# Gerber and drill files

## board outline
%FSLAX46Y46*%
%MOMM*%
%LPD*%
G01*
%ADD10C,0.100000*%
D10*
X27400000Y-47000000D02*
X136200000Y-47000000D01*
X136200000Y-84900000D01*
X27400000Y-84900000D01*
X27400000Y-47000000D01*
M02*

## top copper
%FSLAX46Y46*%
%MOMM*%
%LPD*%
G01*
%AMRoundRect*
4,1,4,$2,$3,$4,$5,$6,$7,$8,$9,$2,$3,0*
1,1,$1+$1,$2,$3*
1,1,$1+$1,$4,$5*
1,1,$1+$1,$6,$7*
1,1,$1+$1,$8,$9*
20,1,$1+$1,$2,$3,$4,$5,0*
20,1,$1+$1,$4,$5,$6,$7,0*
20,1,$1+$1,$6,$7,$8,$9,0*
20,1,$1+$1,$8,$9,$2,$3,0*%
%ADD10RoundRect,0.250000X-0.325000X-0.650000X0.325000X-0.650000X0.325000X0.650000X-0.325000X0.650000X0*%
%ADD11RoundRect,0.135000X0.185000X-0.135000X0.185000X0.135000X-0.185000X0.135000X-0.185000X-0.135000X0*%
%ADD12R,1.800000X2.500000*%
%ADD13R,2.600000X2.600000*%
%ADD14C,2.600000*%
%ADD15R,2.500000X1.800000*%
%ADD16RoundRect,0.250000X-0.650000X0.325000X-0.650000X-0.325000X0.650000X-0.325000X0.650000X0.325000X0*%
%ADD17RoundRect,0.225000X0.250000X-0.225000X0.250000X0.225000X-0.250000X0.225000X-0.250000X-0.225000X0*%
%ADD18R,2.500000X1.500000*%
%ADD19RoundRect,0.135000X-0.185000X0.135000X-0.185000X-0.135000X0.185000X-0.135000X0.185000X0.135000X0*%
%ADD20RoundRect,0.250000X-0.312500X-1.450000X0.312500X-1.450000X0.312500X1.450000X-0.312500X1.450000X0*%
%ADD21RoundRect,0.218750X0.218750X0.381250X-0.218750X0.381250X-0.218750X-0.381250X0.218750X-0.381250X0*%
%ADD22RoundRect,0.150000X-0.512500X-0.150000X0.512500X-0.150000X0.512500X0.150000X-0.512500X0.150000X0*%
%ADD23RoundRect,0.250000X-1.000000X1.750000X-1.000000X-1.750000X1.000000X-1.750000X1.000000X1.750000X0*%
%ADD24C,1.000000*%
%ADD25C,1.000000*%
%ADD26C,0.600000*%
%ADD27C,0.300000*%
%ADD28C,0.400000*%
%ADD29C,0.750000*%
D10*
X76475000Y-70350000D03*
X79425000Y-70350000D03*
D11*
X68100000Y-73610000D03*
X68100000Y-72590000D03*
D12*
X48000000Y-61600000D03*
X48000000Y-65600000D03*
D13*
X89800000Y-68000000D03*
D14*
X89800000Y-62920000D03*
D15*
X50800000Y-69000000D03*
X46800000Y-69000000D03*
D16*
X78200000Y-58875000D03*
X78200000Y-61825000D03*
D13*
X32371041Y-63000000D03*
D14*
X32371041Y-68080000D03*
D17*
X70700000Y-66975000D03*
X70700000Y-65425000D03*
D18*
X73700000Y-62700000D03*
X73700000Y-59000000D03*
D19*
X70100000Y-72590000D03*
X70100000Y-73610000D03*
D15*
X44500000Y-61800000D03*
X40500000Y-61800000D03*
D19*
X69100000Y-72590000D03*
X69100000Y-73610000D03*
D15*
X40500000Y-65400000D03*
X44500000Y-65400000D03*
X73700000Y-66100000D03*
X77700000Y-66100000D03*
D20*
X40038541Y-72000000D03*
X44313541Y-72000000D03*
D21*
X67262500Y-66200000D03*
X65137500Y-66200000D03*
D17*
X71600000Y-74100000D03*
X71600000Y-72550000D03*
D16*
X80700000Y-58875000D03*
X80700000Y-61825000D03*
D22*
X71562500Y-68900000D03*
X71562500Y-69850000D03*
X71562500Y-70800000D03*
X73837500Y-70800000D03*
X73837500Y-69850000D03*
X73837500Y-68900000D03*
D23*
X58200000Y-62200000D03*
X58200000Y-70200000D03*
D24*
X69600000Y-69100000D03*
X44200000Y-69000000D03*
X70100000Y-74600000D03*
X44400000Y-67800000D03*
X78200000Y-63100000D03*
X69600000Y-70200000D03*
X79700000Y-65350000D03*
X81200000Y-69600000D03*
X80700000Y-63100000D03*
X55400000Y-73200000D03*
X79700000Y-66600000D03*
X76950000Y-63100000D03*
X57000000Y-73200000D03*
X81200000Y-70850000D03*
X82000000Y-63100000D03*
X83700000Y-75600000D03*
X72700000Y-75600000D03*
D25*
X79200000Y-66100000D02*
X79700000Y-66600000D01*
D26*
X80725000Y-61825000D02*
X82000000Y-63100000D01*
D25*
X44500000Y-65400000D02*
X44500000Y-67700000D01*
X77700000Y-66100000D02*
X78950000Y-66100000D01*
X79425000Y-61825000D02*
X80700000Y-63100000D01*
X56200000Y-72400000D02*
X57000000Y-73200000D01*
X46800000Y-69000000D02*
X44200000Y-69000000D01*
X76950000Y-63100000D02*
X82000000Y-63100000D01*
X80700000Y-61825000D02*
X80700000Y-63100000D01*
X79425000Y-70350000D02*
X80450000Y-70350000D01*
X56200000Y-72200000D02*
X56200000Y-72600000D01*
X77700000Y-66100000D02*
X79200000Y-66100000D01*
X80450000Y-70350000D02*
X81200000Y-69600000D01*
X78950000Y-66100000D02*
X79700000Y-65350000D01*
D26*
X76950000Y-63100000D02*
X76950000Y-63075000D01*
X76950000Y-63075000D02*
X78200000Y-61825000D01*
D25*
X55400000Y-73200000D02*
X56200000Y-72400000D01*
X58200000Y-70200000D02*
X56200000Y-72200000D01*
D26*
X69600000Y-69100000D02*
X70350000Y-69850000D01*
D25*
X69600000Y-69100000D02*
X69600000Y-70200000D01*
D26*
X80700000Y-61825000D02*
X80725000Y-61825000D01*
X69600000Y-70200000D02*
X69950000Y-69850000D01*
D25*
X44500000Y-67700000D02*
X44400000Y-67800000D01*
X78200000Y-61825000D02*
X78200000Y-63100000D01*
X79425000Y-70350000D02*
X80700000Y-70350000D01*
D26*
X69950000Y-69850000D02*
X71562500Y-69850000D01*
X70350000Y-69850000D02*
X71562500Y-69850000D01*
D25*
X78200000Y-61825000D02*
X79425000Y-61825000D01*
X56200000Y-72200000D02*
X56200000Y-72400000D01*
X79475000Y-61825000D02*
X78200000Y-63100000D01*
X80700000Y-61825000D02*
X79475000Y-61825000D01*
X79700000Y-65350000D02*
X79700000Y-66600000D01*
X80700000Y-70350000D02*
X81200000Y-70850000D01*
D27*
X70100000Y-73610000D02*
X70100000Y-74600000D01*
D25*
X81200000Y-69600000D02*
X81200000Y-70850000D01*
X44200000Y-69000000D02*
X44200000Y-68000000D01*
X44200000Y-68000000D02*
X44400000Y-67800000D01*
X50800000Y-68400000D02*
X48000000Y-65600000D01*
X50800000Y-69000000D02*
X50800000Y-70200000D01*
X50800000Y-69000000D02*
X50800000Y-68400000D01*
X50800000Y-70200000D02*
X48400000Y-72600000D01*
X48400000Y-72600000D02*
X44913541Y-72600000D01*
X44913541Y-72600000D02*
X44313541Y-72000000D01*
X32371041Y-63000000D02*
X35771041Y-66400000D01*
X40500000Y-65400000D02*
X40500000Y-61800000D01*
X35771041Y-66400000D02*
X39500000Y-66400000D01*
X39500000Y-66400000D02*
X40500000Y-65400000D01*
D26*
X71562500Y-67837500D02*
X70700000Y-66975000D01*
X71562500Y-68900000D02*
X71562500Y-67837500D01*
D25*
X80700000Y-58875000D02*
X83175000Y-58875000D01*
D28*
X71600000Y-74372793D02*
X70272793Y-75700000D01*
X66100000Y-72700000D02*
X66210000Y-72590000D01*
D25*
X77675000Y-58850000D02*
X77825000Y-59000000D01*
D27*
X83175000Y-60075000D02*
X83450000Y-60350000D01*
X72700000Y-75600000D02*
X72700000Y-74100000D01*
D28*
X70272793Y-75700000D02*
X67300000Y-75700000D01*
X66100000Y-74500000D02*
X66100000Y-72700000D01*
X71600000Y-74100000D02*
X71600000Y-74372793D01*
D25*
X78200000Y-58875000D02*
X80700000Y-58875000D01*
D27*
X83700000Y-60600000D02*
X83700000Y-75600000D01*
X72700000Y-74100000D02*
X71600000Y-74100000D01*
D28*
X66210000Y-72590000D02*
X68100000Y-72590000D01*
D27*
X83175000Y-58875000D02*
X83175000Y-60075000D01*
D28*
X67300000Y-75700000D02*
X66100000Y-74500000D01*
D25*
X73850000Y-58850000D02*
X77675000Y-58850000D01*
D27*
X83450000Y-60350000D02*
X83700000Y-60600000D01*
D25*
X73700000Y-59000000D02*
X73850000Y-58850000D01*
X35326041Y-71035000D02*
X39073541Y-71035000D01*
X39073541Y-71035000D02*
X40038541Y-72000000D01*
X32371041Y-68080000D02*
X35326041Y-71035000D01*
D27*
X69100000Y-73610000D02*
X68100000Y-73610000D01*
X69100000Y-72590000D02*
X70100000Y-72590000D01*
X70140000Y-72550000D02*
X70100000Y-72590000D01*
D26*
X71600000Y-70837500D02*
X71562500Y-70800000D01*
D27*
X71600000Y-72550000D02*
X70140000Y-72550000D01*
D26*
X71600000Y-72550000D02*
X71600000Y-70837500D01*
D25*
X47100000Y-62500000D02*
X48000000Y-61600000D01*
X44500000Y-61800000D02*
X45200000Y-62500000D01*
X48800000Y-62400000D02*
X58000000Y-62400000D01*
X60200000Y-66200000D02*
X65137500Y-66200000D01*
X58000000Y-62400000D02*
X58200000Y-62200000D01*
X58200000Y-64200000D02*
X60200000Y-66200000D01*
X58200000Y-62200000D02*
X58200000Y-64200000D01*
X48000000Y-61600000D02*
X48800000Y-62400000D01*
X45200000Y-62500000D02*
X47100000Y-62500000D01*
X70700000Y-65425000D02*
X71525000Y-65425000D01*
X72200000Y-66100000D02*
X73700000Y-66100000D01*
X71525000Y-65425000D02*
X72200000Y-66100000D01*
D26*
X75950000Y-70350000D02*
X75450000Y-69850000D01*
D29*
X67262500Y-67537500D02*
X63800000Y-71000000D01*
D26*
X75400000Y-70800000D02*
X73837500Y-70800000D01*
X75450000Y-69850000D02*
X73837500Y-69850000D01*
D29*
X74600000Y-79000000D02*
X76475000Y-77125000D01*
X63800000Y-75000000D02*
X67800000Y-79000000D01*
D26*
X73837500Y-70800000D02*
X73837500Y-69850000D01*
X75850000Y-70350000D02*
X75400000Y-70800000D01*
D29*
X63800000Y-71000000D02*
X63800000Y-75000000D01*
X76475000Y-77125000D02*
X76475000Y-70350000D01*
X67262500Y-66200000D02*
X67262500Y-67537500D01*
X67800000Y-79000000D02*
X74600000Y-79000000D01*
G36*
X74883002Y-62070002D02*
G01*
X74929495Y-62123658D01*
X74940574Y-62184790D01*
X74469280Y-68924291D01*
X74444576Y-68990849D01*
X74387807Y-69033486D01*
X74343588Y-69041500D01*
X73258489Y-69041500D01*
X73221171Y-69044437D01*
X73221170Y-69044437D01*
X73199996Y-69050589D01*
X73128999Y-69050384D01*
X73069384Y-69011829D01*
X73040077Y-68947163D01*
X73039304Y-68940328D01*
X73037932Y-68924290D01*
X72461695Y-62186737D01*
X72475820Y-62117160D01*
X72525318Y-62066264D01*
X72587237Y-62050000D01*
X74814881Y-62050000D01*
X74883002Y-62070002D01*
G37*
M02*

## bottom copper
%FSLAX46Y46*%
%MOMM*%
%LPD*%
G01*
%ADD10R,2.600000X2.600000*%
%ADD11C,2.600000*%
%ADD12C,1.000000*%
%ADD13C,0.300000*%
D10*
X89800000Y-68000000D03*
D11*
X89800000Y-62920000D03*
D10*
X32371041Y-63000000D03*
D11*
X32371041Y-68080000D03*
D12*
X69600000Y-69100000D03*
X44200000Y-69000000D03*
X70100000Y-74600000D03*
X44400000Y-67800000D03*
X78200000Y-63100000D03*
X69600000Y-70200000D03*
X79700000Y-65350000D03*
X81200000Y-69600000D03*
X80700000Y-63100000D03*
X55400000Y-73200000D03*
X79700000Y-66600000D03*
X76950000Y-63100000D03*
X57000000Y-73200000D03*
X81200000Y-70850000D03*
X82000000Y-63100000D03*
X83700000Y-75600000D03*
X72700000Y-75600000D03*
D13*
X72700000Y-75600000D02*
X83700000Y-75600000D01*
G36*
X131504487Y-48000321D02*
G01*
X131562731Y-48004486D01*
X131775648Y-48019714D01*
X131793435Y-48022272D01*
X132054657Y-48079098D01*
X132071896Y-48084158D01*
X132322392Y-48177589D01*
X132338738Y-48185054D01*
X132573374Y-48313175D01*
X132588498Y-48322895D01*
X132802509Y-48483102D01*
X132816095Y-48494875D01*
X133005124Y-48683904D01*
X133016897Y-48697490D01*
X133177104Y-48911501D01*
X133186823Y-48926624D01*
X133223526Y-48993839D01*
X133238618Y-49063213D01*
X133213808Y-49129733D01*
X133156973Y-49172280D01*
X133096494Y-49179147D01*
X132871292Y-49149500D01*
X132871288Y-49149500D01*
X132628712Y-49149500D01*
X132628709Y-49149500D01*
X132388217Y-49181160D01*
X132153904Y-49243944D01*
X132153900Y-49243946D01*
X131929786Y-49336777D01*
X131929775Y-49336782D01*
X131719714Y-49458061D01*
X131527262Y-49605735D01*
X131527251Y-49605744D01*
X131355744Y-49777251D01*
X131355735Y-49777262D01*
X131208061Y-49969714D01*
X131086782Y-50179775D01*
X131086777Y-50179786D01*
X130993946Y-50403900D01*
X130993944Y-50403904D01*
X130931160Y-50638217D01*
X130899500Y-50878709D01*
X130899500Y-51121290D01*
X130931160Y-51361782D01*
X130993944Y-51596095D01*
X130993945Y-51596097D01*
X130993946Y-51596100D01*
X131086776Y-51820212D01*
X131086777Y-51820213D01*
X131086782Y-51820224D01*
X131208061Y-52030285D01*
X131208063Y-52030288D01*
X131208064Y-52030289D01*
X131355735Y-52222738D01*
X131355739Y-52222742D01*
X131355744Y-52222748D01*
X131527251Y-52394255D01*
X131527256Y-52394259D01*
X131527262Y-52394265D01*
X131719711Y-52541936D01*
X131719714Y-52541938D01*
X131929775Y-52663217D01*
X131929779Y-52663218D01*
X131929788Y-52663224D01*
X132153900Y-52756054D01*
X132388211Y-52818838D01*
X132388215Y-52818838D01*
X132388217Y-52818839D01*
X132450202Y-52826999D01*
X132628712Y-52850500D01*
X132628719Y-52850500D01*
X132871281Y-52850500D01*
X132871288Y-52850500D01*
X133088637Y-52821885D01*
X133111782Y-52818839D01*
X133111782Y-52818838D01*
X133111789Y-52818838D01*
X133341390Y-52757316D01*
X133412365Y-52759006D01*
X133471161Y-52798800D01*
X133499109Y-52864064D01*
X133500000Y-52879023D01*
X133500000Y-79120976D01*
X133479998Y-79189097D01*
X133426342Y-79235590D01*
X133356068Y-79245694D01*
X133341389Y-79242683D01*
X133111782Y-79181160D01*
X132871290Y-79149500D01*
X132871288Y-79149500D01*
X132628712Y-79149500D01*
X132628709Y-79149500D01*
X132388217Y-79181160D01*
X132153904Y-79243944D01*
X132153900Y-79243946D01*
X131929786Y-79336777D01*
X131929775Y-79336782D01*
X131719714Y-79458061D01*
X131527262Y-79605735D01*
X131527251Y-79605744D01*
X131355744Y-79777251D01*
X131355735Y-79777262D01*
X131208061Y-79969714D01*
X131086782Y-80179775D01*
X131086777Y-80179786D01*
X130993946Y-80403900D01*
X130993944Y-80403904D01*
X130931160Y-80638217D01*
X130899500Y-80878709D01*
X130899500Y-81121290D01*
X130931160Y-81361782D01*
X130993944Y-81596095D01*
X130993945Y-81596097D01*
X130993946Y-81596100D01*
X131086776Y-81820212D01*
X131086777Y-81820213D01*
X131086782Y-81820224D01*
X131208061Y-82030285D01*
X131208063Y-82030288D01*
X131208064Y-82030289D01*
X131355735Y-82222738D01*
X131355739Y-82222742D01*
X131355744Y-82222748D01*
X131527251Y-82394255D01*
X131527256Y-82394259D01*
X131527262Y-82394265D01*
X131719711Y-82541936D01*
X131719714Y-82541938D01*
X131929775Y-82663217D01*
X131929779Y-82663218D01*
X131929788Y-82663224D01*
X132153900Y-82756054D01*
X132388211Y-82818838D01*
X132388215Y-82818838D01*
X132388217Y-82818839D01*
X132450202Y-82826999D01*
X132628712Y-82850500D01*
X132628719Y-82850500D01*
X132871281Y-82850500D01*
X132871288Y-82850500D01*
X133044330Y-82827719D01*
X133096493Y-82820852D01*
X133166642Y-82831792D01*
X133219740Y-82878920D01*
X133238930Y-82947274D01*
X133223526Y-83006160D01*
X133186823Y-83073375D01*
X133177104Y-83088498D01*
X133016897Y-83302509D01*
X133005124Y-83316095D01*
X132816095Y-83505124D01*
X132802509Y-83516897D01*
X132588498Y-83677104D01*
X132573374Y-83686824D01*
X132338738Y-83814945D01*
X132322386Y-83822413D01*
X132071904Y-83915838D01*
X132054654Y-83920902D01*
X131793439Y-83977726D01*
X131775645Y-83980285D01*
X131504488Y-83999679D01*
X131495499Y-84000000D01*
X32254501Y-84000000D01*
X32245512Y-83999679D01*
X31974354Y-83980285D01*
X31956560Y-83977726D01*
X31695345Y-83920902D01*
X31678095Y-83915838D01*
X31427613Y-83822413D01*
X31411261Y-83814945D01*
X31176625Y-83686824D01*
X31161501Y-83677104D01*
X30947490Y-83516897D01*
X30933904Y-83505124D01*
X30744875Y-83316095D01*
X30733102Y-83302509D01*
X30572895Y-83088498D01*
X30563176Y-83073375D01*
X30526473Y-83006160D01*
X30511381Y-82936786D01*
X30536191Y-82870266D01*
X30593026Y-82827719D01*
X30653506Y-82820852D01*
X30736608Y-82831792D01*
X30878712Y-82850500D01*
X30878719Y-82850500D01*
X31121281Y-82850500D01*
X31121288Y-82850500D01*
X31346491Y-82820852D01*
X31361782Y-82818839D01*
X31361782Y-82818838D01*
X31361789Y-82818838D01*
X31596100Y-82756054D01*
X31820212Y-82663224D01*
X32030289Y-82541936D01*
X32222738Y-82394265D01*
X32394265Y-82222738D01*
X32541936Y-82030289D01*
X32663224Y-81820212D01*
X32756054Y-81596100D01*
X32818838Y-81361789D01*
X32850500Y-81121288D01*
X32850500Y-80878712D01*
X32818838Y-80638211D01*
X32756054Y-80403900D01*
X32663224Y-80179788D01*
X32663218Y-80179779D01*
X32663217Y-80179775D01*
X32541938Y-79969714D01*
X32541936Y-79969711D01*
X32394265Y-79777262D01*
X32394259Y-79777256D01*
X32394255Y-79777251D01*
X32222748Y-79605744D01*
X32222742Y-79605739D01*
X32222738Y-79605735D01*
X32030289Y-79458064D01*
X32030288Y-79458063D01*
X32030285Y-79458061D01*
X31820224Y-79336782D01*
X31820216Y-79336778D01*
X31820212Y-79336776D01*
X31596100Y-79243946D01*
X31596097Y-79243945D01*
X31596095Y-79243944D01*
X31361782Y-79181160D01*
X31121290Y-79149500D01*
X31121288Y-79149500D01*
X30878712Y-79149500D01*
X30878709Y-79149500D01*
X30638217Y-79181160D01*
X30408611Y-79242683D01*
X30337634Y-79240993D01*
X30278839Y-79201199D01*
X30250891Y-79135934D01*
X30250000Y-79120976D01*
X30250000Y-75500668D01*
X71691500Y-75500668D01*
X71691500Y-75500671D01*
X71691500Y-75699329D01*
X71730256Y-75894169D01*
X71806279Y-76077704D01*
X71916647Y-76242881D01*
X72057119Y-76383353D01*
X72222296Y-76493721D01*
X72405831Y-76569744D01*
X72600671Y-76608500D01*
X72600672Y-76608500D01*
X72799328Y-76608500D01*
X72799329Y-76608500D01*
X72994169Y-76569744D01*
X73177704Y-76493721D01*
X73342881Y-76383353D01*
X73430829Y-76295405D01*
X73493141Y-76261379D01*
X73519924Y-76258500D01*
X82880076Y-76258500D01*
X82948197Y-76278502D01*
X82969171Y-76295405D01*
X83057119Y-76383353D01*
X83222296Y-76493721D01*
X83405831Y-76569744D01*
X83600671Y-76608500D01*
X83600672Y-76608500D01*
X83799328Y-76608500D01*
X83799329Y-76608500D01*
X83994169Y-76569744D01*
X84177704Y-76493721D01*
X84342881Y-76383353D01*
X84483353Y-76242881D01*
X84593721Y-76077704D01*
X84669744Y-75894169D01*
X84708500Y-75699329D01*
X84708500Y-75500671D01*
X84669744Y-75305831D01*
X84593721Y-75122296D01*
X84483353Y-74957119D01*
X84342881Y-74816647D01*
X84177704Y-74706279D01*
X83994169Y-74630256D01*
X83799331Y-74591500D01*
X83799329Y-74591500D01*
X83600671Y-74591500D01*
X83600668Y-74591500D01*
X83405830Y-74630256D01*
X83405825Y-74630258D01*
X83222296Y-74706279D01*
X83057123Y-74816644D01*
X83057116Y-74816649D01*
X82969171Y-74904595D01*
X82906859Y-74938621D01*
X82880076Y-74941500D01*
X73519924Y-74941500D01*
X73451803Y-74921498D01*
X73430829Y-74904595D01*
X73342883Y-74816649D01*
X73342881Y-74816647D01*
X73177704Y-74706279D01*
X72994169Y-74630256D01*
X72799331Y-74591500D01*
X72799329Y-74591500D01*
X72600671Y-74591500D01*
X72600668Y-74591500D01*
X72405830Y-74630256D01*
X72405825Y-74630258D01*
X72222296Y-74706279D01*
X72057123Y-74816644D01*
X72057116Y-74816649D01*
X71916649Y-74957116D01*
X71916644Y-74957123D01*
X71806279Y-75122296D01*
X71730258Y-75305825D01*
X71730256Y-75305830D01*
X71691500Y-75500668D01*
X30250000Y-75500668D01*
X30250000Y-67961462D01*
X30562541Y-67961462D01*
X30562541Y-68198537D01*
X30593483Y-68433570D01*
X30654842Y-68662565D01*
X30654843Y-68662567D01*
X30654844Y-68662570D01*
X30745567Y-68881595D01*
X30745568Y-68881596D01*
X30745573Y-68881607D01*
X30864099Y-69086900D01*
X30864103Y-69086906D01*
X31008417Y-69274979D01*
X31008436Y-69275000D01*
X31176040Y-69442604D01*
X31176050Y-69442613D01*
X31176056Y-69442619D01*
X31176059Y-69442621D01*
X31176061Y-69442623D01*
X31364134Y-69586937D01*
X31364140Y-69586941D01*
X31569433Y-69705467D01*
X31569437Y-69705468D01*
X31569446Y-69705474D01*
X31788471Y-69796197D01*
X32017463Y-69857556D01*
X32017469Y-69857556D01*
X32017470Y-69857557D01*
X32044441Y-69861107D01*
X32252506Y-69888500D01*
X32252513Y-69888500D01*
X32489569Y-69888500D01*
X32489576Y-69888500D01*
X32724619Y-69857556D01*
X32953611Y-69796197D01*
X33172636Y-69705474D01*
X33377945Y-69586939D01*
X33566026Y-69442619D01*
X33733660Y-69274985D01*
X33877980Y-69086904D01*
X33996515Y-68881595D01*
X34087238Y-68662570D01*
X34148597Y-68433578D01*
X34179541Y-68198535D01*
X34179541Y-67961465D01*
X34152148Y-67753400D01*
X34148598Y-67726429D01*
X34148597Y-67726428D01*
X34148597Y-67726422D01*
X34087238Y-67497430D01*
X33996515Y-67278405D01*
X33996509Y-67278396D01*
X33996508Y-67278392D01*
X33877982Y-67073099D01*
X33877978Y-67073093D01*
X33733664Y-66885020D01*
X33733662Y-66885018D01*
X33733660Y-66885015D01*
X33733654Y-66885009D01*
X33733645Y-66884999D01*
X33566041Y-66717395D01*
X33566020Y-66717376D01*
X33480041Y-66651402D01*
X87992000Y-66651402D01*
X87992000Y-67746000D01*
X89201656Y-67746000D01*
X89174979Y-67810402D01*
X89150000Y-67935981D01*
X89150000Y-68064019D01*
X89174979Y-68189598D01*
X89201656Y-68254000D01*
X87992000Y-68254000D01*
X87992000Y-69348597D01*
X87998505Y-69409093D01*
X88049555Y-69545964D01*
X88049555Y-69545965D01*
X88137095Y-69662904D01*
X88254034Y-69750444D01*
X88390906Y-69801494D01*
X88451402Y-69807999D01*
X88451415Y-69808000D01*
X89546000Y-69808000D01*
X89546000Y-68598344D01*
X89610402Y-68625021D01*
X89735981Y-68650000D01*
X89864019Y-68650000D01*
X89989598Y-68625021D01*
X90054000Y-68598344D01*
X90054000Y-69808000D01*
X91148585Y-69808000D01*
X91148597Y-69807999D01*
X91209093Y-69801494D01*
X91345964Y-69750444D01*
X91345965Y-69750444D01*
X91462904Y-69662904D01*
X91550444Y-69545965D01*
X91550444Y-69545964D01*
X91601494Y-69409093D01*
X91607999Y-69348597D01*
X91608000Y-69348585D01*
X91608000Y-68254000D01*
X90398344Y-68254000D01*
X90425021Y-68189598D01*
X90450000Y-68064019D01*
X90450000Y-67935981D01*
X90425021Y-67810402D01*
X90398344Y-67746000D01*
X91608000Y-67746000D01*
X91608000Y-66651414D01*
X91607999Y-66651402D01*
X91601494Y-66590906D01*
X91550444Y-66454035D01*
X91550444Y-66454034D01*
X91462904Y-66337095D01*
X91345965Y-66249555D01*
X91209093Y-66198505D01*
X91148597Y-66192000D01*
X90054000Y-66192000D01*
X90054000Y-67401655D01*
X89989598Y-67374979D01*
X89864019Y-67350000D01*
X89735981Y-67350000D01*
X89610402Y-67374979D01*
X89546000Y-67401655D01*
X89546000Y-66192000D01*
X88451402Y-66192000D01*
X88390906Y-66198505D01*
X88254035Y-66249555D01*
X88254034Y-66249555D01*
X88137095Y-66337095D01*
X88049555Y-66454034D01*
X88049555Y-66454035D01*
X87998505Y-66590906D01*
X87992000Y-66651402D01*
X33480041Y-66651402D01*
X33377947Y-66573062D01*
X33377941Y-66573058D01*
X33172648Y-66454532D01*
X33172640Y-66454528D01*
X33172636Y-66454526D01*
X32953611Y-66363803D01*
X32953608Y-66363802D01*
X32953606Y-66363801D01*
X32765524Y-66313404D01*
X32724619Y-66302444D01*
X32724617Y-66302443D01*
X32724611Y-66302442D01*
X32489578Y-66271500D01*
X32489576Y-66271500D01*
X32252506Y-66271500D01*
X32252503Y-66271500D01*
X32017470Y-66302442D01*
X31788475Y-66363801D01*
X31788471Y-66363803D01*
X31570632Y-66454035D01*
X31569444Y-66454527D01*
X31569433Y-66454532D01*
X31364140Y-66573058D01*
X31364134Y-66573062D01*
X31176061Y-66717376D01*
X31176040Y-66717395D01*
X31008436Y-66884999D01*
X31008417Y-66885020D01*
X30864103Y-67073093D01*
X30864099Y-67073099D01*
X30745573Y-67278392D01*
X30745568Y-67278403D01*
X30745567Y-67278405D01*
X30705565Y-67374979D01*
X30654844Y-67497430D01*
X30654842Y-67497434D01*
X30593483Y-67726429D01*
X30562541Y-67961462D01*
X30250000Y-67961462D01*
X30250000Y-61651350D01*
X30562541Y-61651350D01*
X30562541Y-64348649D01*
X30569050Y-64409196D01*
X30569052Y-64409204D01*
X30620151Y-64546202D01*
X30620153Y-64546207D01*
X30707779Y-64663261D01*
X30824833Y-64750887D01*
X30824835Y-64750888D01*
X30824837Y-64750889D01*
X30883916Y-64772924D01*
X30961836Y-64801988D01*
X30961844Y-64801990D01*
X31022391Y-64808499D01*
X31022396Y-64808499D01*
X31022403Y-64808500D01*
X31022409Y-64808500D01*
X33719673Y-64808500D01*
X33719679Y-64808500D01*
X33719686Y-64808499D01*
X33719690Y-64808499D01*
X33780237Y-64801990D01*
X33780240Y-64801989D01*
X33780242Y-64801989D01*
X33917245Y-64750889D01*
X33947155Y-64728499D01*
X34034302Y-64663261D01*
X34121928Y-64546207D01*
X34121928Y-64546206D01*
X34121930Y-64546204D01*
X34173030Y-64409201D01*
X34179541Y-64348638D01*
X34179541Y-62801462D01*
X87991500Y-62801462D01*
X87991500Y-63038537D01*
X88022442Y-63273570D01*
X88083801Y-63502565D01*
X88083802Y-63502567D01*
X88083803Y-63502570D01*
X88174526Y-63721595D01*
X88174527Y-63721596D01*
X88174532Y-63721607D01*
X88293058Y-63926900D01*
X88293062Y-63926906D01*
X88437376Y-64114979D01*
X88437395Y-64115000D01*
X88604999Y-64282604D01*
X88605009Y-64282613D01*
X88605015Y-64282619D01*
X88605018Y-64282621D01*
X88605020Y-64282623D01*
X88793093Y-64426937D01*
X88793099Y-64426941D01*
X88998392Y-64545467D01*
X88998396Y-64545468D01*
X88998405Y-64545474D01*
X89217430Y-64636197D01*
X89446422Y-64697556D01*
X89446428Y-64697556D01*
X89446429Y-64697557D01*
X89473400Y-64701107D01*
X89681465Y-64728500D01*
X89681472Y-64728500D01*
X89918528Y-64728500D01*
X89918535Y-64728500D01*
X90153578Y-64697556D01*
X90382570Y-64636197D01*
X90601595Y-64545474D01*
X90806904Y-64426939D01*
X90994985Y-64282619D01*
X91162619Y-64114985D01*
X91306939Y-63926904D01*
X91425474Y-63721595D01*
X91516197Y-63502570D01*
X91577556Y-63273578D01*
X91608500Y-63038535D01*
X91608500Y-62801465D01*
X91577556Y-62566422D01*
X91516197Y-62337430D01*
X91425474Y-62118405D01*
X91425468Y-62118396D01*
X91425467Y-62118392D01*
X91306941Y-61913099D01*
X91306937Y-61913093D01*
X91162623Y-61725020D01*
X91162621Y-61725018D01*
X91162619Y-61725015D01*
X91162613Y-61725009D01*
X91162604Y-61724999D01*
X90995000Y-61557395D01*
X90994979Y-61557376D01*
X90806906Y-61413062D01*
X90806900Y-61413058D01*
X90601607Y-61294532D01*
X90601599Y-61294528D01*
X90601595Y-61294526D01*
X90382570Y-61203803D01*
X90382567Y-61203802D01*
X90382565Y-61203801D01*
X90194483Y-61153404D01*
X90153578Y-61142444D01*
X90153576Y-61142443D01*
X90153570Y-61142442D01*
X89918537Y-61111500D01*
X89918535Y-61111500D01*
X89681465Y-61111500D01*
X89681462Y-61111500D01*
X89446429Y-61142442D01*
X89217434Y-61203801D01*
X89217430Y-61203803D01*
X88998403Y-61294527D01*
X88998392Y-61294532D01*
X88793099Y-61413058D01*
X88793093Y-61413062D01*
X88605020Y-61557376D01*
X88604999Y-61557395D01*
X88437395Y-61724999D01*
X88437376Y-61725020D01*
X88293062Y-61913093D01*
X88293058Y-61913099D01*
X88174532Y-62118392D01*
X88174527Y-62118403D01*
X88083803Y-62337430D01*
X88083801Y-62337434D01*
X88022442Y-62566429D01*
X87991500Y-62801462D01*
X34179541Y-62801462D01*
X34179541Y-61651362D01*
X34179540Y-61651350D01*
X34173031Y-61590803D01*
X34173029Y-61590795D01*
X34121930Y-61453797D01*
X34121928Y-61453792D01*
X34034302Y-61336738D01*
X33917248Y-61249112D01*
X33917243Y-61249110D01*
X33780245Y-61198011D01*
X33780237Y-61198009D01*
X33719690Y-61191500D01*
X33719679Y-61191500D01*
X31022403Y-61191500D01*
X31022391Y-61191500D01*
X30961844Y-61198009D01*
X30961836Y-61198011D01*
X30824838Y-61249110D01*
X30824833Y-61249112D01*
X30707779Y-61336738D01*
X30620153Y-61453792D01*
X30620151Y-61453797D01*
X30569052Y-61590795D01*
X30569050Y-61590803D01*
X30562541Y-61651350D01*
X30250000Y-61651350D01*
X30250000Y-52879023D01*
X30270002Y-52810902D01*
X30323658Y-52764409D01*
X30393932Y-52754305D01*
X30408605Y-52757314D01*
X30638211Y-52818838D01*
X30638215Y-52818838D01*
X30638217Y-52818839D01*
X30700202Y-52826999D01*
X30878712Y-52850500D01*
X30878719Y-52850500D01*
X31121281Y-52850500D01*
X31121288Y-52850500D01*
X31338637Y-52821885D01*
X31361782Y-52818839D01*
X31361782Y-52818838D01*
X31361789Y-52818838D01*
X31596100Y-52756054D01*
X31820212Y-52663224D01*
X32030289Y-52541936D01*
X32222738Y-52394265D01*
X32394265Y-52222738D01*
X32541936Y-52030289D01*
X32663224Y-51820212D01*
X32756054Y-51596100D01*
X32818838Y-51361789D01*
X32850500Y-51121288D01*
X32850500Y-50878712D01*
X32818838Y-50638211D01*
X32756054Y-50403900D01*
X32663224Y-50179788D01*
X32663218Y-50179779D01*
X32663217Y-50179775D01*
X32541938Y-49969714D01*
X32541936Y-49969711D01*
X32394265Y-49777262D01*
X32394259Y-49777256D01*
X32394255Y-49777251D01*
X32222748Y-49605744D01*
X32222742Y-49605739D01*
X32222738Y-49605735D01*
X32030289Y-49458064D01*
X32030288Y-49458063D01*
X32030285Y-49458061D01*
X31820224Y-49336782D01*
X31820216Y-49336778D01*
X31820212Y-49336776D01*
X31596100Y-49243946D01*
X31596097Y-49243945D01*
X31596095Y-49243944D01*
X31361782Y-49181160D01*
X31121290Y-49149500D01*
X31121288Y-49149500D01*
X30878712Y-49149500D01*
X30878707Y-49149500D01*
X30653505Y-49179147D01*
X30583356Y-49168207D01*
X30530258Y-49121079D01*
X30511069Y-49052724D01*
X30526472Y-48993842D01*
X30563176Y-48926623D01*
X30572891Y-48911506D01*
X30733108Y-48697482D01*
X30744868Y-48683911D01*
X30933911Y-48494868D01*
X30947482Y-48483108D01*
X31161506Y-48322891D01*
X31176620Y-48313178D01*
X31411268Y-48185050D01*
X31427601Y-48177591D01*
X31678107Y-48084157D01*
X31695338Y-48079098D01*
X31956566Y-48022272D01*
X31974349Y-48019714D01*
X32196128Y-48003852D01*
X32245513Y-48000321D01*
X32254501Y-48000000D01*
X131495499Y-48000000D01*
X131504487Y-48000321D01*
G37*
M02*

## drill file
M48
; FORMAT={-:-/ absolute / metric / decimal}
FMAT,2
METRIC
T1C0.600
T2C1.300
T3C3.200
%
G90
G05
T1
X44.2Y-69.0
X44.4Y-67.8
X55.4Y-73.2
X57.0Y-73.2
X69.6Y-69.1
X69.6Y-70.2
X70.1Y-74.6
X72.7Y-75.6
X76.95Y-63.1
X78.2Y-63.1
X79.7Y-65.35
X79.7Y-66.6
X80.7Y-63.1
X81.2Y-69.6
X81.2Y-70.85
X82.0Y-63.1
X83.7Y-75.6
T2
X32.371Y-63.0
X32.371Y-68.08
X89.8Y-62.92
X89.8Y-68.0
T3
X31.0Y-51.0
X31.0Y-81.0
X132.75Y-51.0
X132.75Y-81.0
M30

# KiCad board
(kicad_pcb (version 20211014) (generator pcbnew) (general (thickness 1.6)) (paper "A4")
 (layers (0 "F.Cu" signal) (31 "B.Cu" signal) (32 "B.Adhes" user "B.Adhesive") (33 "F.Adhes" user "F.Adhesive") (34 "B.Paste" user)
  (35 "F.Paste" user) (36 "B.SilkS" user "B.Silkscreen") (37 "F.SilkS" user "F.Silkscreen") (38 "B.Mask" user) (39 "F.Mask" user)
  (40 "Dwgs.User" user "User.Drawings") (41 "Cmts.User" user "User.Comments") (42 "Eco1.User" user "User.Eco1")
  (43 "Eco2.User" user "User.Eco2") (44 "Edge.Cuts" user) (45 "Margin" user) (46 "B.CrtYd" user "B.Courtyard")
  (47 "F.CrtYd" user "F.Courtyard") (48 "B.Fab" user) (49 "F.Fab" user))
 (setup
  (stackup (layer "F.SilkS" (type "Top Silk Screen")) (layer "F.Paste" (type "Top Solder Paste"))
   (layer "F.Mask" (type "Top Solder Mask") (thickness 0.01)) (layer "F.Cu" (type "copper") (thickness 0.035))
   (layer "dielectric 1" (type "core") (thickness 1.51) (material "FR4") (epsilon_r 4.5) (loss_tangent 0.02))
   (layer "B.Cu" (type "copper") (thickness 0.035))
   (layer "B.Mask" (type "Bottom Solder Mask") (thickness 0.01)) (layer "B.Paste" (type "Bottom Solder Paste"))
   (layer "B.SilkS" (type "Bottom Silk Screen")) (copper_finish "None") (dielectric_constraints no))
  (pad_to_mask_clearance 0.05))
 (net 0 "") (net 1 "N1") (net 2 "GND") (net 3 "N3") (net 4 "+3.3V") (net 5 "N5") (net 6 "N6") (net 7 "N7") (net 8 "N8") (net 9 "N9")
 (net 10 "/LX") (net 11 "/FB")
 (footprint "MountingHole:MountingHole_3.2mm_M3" (layer "F.Cu") (at 132.75 51)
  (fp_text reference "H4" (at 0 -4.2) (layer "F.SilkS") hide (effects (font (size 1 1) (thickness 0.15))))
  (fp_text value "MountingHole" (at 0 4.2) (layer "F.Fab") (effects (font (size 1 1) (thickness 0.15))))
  (pad "" np_thru_hole circle (at 0 0) (size 3.2 3.2) (drill 3.2) (layers *.Cu *.Mask)))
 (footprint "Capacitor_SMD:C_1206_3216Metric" (layer "F.Cu") (at 77.95 70.35)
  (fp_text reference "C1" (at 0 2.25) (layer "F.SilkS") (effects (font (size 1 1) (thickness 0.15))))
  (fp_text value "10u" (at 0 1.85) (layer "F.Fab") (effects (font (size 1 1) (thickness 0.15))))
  (pad "1" smd roundrect (at -1.475 0) (size 1.15 1.8) (layers "F.Cu" "F.Paste" "F.Mask") (roundrect_rratio 0.217391) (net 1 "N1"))
  (pad "2" smd roundrect (at 1.475 0) (size 1.15 1.8) (layers "F.Cu" "F.Paste" "F.Mask") (roundrect_rratio 0.217391) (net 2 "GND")))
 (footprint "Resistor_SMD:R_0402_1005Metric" (layer "F.Cu") (at 68.1 73.1 90)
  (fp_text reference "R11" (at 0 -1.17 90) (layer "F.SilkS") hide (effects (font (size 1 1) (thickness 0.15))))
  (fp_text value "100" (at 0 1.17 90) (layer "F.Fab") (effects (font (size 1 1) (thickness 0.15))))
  (pad "1" smd roundrect (at -0.51 0 90) (size 0.54 0.64) (layers "F.Cu" "F.Paste" "F.Mask") (roundrect_rratio 0.25) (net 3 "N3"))
  (pad "2" smd roundrect (at 0.51 0 90) (size 0.54 0.64) (layers "F.Cu" "F.Paste" "F.Mask") (roundrect_rratio 0.25) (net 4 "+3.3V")))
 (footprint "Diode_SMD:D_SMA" (layer "F.Cu") (at 48 63.6 -90)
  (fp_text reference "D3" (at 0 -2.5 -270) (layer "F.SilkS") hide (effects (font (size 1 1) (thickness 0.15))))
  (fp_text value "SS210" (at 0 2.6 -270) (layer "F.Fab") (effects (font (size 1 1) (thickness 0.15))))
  (pad "1" smd rect (at -2 0 270) (size 2.5 1.8) (layers "F.Cu" "F.Paste" "F.Mask") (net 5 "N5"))
  (pad "2" smd rect (at 2 0 270) (size 2.5 1.8) (layers "F.Cu" "F.Paste" "F.Mask") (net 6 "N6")))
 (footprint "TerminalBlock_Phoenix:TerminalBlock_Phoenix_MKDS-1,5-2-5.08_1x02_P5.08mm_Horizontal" (layer "F.Cu") (at 89.8 68 90)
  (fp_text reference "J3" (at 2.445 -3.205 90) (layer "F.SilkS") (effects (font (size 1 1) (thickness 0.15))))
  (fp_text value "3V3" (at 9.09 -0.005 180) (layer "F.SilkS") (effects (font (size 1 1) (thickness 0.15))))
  (pad "1" thru_hole rect (at 0 0 90) (size 2.6 2.6) (drill 1.3) (layers *.Cu *.Mask) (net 2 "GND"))
  (pad "2" thru_hole circle (at 5.08 0 90) (size 2.6 2.6) (drill 1.3) (layers *.Cu *.Mask) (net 4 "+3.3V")))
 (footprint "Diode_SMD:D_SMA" (layer "F.Cu") (at 48.8 69 180)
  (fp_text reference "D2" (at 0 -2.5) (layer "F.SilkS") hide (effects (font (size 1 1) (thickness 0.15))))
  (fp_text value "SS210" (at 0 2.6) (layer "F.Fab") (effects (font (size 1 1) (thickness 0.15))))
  (pad "1" smd rect (at -2 0 180) (size 2.5 1.8) (layers "F.Cu" "F.Paste" "F.Mask") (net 6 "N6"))
  (pad "2" smd rect (at 2 0 180) (size 2.5 1.8) (layers "F.Cu" "F.Paste" "F.Mask") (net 2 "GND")))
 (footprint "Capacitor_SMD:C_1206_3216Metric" (layer "F.Cu") (at 78.2 60.35 -90)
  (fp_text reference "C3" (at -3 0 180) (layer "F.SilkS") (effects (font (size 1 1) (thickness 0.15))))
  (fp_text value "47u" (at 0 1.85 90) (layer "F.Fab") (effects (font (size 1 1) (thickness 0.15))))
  (pad "1" smd roundrect (at -1.475 0 270) (size 1.15 1.8) (layers "F.Cu" "F.Paste" "F.Mask") (roundrect_rratio 0.217391) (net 4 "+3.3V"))
  (pad "2" smd roundrect (at 1.475 0 270) (size 1.15 1.8) (layers "F.Cu" "F.Paste" "F.Mask") (roundrect_rratio 0.217391) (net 2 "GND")))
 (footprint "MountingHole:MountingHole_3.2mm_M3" (layer "F.Cu") (at 31 51)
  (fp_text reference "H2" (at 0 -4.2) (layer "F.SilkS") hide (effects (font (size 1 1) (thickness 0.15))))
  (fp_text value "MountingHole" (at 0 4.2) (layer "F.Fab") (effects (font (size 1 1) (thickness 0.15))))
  (pad "" np_thru_hole circle (at 0 0) (size 3.2 3.2) (drill 3.2) (layers *.Cu *.Mask)))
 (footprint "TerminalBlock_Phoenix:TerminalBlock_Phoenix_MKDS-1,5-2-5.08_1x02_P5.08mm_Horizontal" (layer "F.Cu") (at 32.371041 63 -90)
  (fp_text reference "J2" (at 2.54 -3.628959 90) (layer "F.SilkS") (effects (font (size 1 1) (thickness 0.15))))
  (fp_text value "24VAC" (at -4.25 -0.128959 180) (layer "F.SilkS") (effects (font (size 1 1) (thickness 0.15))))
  (pad "1" thru_hole rect (at 0 0 270) (size 2.6 2.6) (drill 1.3) (layers *.Cu *.Mask) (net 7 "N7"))
  (pad "2" thru_hole circle (at 5.08 0 270) (size 2.6 2.6) (drill 1.3) (layers *.Cu *.Mask) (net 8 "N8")))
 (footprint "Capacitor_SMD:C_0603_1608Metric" (layer "F.Cu") (at 70.7 66.2 90)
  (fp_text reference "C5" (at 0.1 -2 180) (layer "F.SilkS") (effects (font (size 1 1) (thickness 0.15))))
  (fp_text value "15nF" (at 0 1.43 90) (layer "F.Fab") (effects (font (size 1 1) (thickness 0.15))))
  (pad "1" smd roundrect (at -0.775 0 90) (size 0.9 0.95) (layers "F.Cu" "F.Paste" "F.Mask") (roundrect_rratio 0.25) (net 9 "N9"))
  (pad "2" smd roundrect (at 0.775 0 90) (size 0.9 0.95) (layers "F.Cu" "F.Paste" "F.Mask") (roundrect_rratio 0.25) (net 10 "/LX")))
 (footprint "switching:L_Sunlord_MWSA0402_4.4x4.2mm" (layer "F.Cu") (at 73.7 60.85 90)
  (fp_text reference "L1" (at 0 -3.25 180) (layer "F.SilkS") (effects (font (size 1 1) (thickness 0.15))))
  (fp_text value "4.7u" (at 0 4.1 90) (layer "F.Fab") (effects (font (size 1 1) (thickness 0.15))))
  (pad "1" smd rect (at -1.85 0 90) (size 1.5 2.5) (layers "F.Cu" "F.Paste" "F.Mask") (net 10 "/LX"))
  (pad "2" smd rect (at 1.85 0 90) (size 1.5 2.5) (layers "F.Cu" "F.Paste" "F.Mask") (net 4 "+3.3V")))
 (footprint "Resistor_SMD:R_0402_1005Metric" (layer "F.Cu") (at 70.1 73.1 -90)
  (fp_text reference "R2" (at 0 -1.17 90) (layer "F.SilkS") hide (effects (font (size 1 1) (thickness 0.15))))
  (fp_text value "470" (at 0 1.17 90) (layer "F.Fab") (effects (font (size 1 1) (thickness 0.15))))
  (pad "1" smd roundrect (at -0.51 0 270) (size 0.54 0.64) (layers "F.Cu" "F.Paste" "F.Mask") (roundrect_rratio 0.25) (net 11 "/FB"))
  (pad "2" smd roundrect (at 0.51 0 270) (size 0.54 0.64) (layers "F.Cu" "F.Paste" "F.Mask") (roundrect_rratio 0.25) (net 2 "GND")))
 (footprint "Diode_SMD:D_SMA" (layer "F.Cu") (at 42.5 61.8 180)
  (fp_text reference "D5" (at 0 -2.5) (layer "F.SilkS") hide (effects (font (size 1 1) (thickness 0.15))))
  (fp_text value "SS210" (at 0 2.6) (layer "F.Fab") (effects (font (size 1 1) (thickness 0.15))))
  (pad "1" smd rect (at -2 0 180) (size 2.5 1.8) (layers "F.Cu" "F.Paste" "F.Mask") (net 5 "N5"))
  (pad "2" smd rect (at 2 0 180) (size 2.5 1.8) (layers "F.Cu" "F.Paste" "F.Mask") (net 7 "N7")))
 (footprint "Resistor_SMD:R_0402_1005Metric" (layer "F.Cu") (at 69.1 73.1 -90)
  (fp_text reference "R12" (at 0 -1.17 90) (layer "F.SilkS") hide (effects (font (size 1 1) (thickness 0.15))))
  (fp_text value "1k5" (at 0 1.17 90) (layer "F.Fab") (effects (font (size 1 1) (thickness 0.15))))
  (pad "1" smd roundrect (at -0.51 0 270) (size 0.54 0.64) (layers "F.Cu" "F.Paste" "F.Mask") (roundrect_rratio 0.25) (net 11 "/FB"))
  (pad "2" smd roundrect (at 0.51 0 270) (size 0.54 0.64) (layers "F.Cu" "F.Paste" "F.Mask") (roundrect_rratio 0.25) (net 3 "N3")))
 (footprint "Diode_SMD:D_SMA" (layer "F.Cu") (at 42.5 65.4)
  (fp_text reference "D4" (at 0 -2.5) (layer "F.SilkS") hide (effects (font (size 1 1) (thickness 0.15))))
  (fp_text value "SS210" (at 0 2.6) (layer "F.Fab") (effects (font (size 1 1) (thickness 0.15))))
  (pad "1" smd rect (at -2 0) (size 2.5 1.8) (layers "F.Cu" "F.Paste" "F.Mask") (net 7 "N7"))
  (pad "2" smd rect (at 2 0) (size 2.5 1.8) (layers "F.Cu" "F.Paste" "F.Mask") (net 2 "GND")))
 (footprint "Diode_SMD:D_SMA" (layer "F.Cu") (at 75.7 66.1)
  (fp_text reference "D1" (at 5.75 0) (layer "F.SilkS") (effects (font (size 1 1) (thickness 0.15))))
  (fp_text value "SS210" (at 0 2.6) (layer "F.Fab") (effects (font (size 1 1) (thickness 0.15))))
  (pad "1" smd rect (at -2 0) (size 2.5 1.8) (layers "F.Cu" "F.Paste" "F.Mask") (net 10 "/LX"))
  (pad "2" smd rect (at 2 0) (size 2.5 1.8) (layers "F.Cu" "F.Paste" "F.Mask") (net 2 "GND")))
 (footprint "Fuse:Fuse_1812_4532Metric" (layer "F.Cu") (at 42.176041 72)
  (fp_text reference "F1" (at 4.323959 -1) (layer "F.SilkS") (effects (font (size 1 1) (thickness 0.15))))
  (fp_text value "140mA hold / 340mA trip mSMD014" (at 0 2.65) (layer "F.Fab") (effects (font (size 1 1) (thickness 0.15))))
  (pad "1" smd roundrect (at -2.1375 0) (size 1.125 3.4) (layers "F.Cu" "F.Paste" "F.Mask") (roundrect_rratio 0.222222) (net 8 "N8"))
  (pad "2" smd roundrect (at 2.1375 0) (size 1.125 3.4) (layers "F.Cu" "F.Paste" "F.Mask") (roundrect_rratio 0.222222) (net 6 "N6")))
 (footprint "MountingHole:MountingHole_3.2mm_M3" (layer "F.Cu") (at 132.75 81)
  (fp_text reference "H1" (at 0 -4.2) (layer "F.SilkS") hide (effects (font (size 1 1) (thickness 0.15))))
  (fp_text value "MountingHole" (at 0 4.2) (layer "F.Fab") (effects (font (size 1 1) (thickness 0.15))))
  (pad "" np_thru_hole circle (at 0 0) (size 3.2 3.2) (drill 3.2) (layers *.Cu *.Mask)))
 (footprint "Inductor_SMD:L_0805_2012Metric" (layer "F.Cu") (at 66.2 66.2 180)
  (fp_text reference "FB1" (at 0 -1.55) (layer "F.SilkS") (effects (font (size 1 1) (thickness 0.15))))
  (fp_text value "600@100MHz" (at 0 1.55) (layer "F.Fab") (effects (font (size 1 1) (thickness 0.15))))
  (pad "1" smd roundrect (at -1.0625 0 180) (size 0.875 1.2) (layers "F.Cu" "F.Paste" "F.Mask") (roundrect_rratio 0.25) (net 1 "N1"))
  (pad "2" smd roundrect (at 1.0625 0 180) (size 0.875 1.2) (layers "F.Cu" "F.Paste" "F.Mask") (roundrect_rratio 0.25) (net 5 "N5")))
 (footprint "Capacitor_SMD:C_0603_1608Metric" (layer "F.Cu") (at 71.6 73.325 90)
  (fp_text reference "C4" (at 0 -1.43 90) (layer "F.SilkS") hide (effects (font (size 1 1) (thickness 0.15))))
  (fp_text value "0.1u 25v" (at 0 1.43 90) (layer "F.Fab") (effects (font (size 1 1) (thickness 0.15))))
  (pad "1" smd roundrect (at -0.775 0 90) (size 0.9 0.95) (layers "F.Cu" "F.Paste" "F.Mask") (roundrect_rratio 0.25) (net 4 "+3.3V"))
  (pad "2" smd roundrect (at 0.775 0 90) (size 0.9 0.95) (layers "F.Cu" "F.Paste" "F.Mask") (roundrect_rratio 0.25) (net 11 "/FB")))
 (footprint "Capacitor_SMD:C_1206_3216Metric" (layer "F.Cu") (at 80.7 60.35 -90)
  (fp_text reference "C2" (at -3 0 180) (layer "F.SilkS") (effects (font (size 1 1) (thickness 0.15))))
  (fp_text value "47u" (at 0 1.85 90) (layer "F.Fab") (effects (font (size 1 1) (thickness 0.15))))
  (pad "1" smd roundrect (at -1.475 0 270) (size 1.15 1.8) (layers "F.Cu" "F.Paste" "F.Mask") (roundrect_rratio 0.217391) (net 4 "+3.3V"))
  (pad "2" smd roundrect (at 1.475 0 270) (size 1.15 1.8) (layers "F.Cu" "F.Paste" "F.Mask") (roundrect_rratio 0.217391) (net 2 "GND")))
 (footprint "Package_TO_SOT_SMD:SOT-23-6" (layer "F.Cu") (at 72.7 69.85)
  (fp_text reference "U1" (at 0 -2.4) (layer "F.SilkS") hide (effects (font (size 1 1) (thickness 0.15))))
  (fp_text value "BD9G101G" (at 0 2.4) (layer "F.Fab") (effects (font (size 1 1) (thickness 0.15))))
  (pad "1" smd roundrect (at -1.1375 -0.95) (size 1.325 0.6) (layers "F.Cu" "F.Paste" "F.Mask") (roundrect_rratio 0.25) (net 9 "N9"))
  (pad "2" smd roundrect (at -1.1375 0) (size 1.325 0.6) (layers "F.Cu" "F.Paste" "F.Mask") (roundrect_rratio 0.25) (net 2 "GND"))
  (pad "3" smd roundrect (at -1.1375 0.95) (size 1.325 0.6) (layers "F.Cu" "F.Paste" "F.Mask") (roundrect_rratio 0.25) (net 11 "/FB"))
  (pad "4" smd roundrect (at 1.1375 0.95) (size 1.325 0.6) (layers "F.Cu" "F.Paste" "F.Mask") (roundrect_rratio 0.25) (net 1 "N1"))
  (pad "5" smd roundrect (at 1.1375 0) (size 1.325 0.6) (layers "F.Cu" "F.Paste" "F.Mask") (roundrect_rratio 0.25) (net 1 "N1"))
  (pad "6" smd roundrect (at 1.1375 -0.95) (size 1.325 0.6) (layers "F.Cu" "F.Paste" "F.Mask") (roundrect_rratio 0.25) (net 10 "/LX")))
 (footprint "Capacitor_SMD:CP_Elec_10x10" (layer "F.Cu") (at 58.2 66.2 -90)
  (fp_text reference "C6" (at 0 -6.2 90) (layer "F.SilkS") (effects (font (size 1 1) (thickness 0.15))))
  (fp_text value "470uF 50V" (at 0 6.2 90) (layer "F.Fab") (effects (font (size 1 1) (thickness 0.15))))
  (pad "1" smd roundrect (at -4 0 270) (size 4 2.5) (layers "F.Cu" "F.Paste" "F.Mask") (roundrect_rratio 0.1) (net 5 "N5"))
  (pad "2" smd roundrect (at 4 0 270) (size 4 2.5) (layers "F.Cu" "F.Paste" "F.Mask") (roundrect_rratio 0.1) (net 2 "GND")))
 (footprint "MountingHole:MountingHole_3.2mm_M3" (layer "F.Cu") (at 31 81)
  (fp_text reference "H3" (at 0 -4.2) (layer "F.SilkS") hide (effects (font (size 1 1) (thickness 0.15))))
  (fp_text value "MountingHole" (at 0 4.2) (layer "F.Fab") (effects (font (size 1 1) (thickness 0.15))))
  (pad "" np_thru_hole circle (at 0 0) (size 3.2 3.2) (drill 3.2) (layers *.Cu *.Mask)))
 (gr_rect (start 27.4 47) (end 136.2 84.9) (layer "Edge.Cuts") (width 0.1) (fill none))
 (segment (start 79.2 66.1) (end 79.7 66.6) (width 1) (layer "F.Cu") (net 2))
 (segment (start 80.725 61.825) (end 82 63.1) (width 0.6) (layer "F.Cu") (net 2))
 (segment (start 44.5 65.4) (end 44.5 67.7) (width 1) (layer "F.Cu") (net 2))
 (segment (start 77.7 66.1) (end 78.95 66.1) (width 1) (layer "F.Cu") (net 2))
 (segment (start 79.425 61.825) (end 80.7 63.1) (width 1) (layer "F.Cu") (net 2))
 (segment (start 56.2 72.4) (end 57 73.2) (width 1) (layer "F.Cu") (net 2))
 (segment (start 46.8 69) (end 44.2 69) (width 1) (layer "F.Cu") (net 2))
 (segment (start 76.95 63.1) (end 82 63.1) (width 1) (layer "F.Cu") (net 2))
 (segment (start 80.7 61.825) (end 80.7 63.1) (width 1) (layer "F.Cu") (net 2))
 (segment (start 79.425 70.35) (end 80.45 70.35) (width 1) (layer "F.Cu") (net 2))
 (segment (start 56.2 72.2) (end 56.2 72.6) (width 1) (layer "F.Cu") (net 2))
 (segment (start 77.7 66.1) (end 79.2 66.1) (width 1) (layer "F.Cu") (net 2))
 (segment (start 80.45 70.35) (end 81.2 69.6) (width 1) (layer "F.Cu") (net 2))
 (segment (start 78.95 66.1) (end 79.7 65.35) (width 1) (layer "F.Cu") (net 2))
 (segment (start 76.95 63.1) (end 76.95 63.075) (width 0.6) (layer "F.Cu") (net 2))
 (segment (start 76.95 63.075) (end 78.2 61.825) (width 0.6) (layer "F.Cu") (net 2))
 (segment (start 55.4 73.2) (end 56.2 72.4) (width 1) (layer "F.Cu") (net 2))
 (segment (start 58.2 70.2) (end 56.2 72.2) (width 1) (layer "F.Cu") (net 2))
 (segment (start 69.6 69.1) (end 70.35 69.85) (width 0.6) (layer "F.Cu") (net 2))
 (segment (start 69.6 69.1) (end 69.6 70.2) (width 1) (layer "F.Cu") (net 2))
 (segment (start 80.7 61.825) (end 80.725 61.825) (width 0.6) (layer "F.Cu") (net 2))
 (segment (start 69.6 70.2) (end 69.95 69.85) (width 0.6) (layer "F.Cu") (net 2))
 (segment (start 44.5 67.7) (end 44.4 67.8) (width 1) (layer "F.Cu") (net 2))
 (segment (start 78.2 61.825) (end 78.2 63.1) (width 1) (layer "F.Cu") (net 2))
 (segment (start 79.425 70.35) (end 80.7 70.35) (width 1) (layer "F.Cu") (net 2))
 (segment (start 69.95 69.85) (end 71.5625 69.85) (width 0.6) (layer "F.Cu") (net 2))
 (segment (start 70.35 69.85) (end 71.5625 69.85) (width 0.6) (layer "F.Cu") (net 2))
 (segment (start 78.2 61.825) (end 79.425 61.825) (width 1) (layer "F.Cu") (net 2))
 (segment (start 56.2 72.2) (end 56.2 72.4) (width 1) (layer "F.Cu") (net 2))
 (segment (start 79.475 61.825) (end 78.2 63.1) (width 1) (layer "F.Cu") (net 2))
 (segment (start 80.7 61.825) (end 79.475 61.825) (width 1) (layer "F.Cu") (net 2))
 (segment (start 79.7 65.35) (end 79.7 66.6) (width 1) (layer "F.Cu") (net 2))
 (segment (start 80.7 70.35) (end 81.2 70.85) (width 1) (layer "F.Cu") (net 2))
 (segment (start 70.1 73.61) (end 70.1 74.6) (width 0.3) (layer "F.Cu") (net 2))
 (segment (start 81.2 69.6) (end 81.2 70.85) (width 1) (layer "F.Cu") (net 2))
 (segment (start 44.2 69) (end 44.2 68) (width 1) (layer "F.Cu") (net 2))
 (segment (start 44.2 68) (end 44.4 67.8) (width 1) (layer "F.Cu") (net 2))
 (via (at 69.6 69.1) (size 1) (drill 0.6) (layers "F.Cu" "B.Cu") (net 2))
 (via (at 44.2 69) (size 1) (drill 0.6) (layers "F.Cu" "B.Cu") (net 2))
 (via (at 70.1 74.6) (size 1) (drill 0.6) (layers "F.Cu" "B.Cu") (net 2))
 (via (at 44.4 67.8) (size 1) (drill 0.6) (layers "F.Cu" "B.Cu") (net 2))
 (via (at 78.2 63.1) (size 1) (drill 0.6) (layers "F.Cu" "B.Cu") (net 2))
 (via (at 69.6 70.2) (size 1) (drill 0.6) (layers "F.Cu" "B.Cu") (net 2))
 (via (at 79.7 65.35) (size 1) (drill 0.6) (layers "F.Cu" "B.Cu") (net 2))
 (via (at 81.2 69.6) (size 1) (drill 0.6) (layers "F.Cu" "B.Cu") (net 2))
 (via (at 80.7 63.1) (size 1) (drill 0.6) (layers "F.Cu" "B.Cu") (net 2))
 (via (at 55.4 73.2) (size 1) (drill 0.6) (layers "F.Cu" "B.Cu") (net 2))
 (via (at 79.7 66.6) (size 1) (drill 0.6) (layers "F.Cu" "B.Cu") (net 2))
 (via (at 76.95 63.1) (size 1) (drill 0.6) (layers "F.Cu" "B.Cu") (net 2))
 (via (at 57 73.2) (size 1) (drill 0.6) (layers "F.Cu" "B.Cu") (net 2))
 (via (at 81.2 70.85) (size 1) (drill 0.6) (layers "F.Cu" "B.Cu") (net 2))
 (via (at 82 63.1) (size 1) (drill 0.6) (layers "F.Cu" "B.Cu") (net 2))
 (segment (start 50.8 68.4) (end 48 65.6) (width 1) (layer "F.Cu") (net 6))
 (segment (start 50.8 69) (end 50.8 70.2) (width 1) (layer "F.Cu") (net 6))
 (segment (start 50.8 69) (end 50.8 68.4) (width 1) (layer "F.Cu") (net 6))
 (segment (start 50.8 70.2) (end 48.4 72.6) (width 1) (layer "F.Cu") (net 6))
 (segment (start 48.4 72.6) (end 44.913541 72.6) (width 1) (layer "F.Cu") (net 6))
 (segment (start 44.913541 72.6) (end 44.313541 72) (width 1) (layer "F.Cu") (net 6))
 (segment (start 32.371041 63) (end 35.771041 66.4) (width 1) (layer "F.Cu") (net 7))
 (segment (start 40.5 65.4) (end 40.5 61.8) (width 1) (layer "F.Cu") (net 7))
 (segment (start 35.771041 66.4) (end 39.5 66.4) (width 1) (layer "F.Cu") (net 7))
 (segment (start 39.5 66.4) (end 40.5 65.4) (width 1) (layer "F.Cu") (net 7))
 (segment (start 71.5625 67.8375) (end 70.7 66.975) (width 0.6) (layer "F.Cu") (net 9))
 (segment (start 71.5625 68.9) (end 71.5625 67.8375) (width 0.6) (layer "F.Cu") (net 9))
 (segment (start 80.7 58.875) (end 83.175 58.875) (width 1) (layer "F.Cu") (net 4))
 (segment (start 71.6 74.372793) (end 70.272793 75.7) (width 0.4) (layer "F.Cu") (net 4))
 (segment (start 66.1 72.7) (end 66.21 72.59) (width 0.4) (layer "F.Cu") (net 4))
 (segment (start 77.675 58.85) (end 77.825 59) (width 1) (layer "F.Cu") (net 4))
 (segment (start 83.175 60.075) (end 83.45 60.35) (width 0.3) (layer "F.Cu") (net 4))
 (segment (start 72.7 75.6) (end 72.7 74.1) (width 0.3) (layer "F.Cu") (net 4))
 (segment (start 70.272793 75.7) (end 67.3 75.7) (width 0.4) (layer "F.Cu") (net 4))
 (segment (start 66.1 74.5) (end 66.1 72.7) (width 0.4) (layer "F.Cu") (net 4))
 (segment (start 71.6 74.1) (end 71.6 74.372793) (width 0.4) (layer "F.Cu") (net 4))
 (segment (start 78.2 58.875) (end 80.7 58.875) (width 1) (layer "F.Cu") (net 4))
 (segment (start 83.7 60.6) (end 83.7 75.6) (width 0.3) (layer "F.Cu") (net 4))
 (segment (start 72.7 74.1) (end 71.6 74.1) (width 0.3) (layer "F.Cu") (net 4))
 (segment (start 66.21 72.59) (end 68.1 72.59) (width 0.4) (layer "F.Cu") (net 4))
 (segment (start 83.175 58.875) (end 83.175 60.075) (width 0.3) (layer "F.Cu") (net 4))
 (segment (start 67.3 75.7) (end 66.1 74.5) (width 0.4) (layer "F.Cu") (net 4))
 (segment (start 73.85 58.85) (end 77.675 58.85) (width 1) (layer "F.Cu") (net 4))
 (segment (start 83.45 60.35) (end 83.7 60.6) (width 0.3) (layer "F.Cu") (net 4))
 (segment (start 73.7 59) (end 73.85 58.85) (width 1) (layer "F.Cu") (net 4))
 (via (at 83.7 75.6) (size 1) (drill 0.6) (layers "F.Cu" "B.Cu") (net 4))
 (via (at 72.7 75.6) (size 1) (drill 0.6) (layers "F.Cu" "B.Cu") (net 4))
 (segment (start 72.7 75.6) (end 83.7 75.6) (width 0.3) (layer "B.Cu") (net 4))
 (segment (start 35.326041 71.035) (end 39.073541 71.035) (width 1) (layer "F.Cu") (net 8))
 (segment (start 39.073541 71.035) (end 40.038541 72) (width 1) (layer "F.Cu") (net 8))
 (segment (start 32.371041 68.08) (end 35.326041 71.035) (width 1) (layer "F.Cu") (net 8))
 (segment (start 69.1 73.61) (end 68.1 73.61) (width 0.3) (layer "F.Cu") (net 3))
 (segment (start 69.1 72.59) (end 70.1 72.59) (width 0.3) (layer "F.Cu") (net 11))
 (segment (start 70.14 72.55) (end 70.1 72.59) (width 0.3) (layer "F.Cu") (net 11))
 (segment (start 71.6 70.8375) (end 71.5625 70.8) (width 0.6) (layer "F.Cu") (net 11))
 (segment (start 71.6 72.55) (end 70.14 72.55) (width 0.3) (layer "F.Cu") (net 11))
 (segment (start 71.6 72.55) (end 71.6 70.8375) (width 0.6) (layer "F.Cu") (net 11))
 (segment (start 47.1 62.5) (end 48 61.6) (width 1) (layer "F.Cu") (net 5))
 (segment (start 44.5 61.8) (end 45.2 62.5) (width 1) (layer "F.Cu") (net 5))
 (segment (start 48.8 62.4) (end 58 62.4) (width 1) (layer "F.Cu") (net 5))
 (segment (start 60.2 66.2) (end 65.1375 66.2) (width 1) (layer "F.Cu") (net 5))
 (segment (start 58 62.4) (end 58.2 62.2) (width 1) (layer "F.Cu") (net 5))
 (segment (start 58.2 64.2) (end 60.2 66.2) (width 1) (layer "F.Cu") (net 5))
 (segment (start 58.2 62.2) (end 58.2 64.2) (width 1) (layer "F.Cu") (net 5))
 (segment (start 48 61.6) (end 48.8 62.4) (width 1) (layer "F.Cu") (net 5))
 (segment (start 45.2 62.5) (end 47.1 62.5) (width 1) (layer "F.Cu") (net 5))
 (segment (start 70.7 65.425) (end 71.525 65.425) (width 1) (layer "F.Cu") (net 10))
 (segment (start 72.2 66.1) (end 73.7 66.1) (width 1) (layer "F.Cu") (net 10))
 (segment (start 71.525 65.425) (end 72.2 66.1) (width 1) (layer "F.Cu") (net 10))
 (segment (start 75.95 70.35) (end 75.45 69.85) (width 0.6) (layer "F.Cu") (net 1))
 (segment (start 67.2625 67.5375) (end 63.8 71) (width 0.75) (layer "F.Cu") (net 1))
 (segment (start 75.4 70.8) (end 73.8375 70.8) (width 0.6) (layer "F.Cu") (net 1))
 (segment (start 75.45 69.85) (end 73.8375 69.85) (width 0.6) (layer "F.Cu") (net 1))
 (segment (start 74.6 79) (end 76.475 77.125) (width 0.75) (layer "F.Cu") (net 1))
 (segment (start 63.8 75) (end 67.8 79) (width 0.75) (layer "F.Cu") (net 1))
 (segment (start 73.8375 70.8) (end 73.8375 69.85) (width 0.6) (layer "F.Cu") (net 1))
 (segment (start 75.85 70.35) (end 75.4 70.8) (width 0.6) (layer "F.Cu") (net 1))
 (segment (start 63.8 71) (end 63.8 75) (width 0.75) (layer "F.Cu") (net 1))
 (segment (start 76.475 77.125) (end 76.475 70.35) (width 0.75) (layer "F.Cu") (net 1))
 (segment (start 67.2625 66.2) (end 67.2625 67.5375) (width 0.75) (layer "F.Cu") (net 1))
 (segment (start 67.8 79) (end 74.6 79) (width 0.75) (layer "F.Cu") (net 1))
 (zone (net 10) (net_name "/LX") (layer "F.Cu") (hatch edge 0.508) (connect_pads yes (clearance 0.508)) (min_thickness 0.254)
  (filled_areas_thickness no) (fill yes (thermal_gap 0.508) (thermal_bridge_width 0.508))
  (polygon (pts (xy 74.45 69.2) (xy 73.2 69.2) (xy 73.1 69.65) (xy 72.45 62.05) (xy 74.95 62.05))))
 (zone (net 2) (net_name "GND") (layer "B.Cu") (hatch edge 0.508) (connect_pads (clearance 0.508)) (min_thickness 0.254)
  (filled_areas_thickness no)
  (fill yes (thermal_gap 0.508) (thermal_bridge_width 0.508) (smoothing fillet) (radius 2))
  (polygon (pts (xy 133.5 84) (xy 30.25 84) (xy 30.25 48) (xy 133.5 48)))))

